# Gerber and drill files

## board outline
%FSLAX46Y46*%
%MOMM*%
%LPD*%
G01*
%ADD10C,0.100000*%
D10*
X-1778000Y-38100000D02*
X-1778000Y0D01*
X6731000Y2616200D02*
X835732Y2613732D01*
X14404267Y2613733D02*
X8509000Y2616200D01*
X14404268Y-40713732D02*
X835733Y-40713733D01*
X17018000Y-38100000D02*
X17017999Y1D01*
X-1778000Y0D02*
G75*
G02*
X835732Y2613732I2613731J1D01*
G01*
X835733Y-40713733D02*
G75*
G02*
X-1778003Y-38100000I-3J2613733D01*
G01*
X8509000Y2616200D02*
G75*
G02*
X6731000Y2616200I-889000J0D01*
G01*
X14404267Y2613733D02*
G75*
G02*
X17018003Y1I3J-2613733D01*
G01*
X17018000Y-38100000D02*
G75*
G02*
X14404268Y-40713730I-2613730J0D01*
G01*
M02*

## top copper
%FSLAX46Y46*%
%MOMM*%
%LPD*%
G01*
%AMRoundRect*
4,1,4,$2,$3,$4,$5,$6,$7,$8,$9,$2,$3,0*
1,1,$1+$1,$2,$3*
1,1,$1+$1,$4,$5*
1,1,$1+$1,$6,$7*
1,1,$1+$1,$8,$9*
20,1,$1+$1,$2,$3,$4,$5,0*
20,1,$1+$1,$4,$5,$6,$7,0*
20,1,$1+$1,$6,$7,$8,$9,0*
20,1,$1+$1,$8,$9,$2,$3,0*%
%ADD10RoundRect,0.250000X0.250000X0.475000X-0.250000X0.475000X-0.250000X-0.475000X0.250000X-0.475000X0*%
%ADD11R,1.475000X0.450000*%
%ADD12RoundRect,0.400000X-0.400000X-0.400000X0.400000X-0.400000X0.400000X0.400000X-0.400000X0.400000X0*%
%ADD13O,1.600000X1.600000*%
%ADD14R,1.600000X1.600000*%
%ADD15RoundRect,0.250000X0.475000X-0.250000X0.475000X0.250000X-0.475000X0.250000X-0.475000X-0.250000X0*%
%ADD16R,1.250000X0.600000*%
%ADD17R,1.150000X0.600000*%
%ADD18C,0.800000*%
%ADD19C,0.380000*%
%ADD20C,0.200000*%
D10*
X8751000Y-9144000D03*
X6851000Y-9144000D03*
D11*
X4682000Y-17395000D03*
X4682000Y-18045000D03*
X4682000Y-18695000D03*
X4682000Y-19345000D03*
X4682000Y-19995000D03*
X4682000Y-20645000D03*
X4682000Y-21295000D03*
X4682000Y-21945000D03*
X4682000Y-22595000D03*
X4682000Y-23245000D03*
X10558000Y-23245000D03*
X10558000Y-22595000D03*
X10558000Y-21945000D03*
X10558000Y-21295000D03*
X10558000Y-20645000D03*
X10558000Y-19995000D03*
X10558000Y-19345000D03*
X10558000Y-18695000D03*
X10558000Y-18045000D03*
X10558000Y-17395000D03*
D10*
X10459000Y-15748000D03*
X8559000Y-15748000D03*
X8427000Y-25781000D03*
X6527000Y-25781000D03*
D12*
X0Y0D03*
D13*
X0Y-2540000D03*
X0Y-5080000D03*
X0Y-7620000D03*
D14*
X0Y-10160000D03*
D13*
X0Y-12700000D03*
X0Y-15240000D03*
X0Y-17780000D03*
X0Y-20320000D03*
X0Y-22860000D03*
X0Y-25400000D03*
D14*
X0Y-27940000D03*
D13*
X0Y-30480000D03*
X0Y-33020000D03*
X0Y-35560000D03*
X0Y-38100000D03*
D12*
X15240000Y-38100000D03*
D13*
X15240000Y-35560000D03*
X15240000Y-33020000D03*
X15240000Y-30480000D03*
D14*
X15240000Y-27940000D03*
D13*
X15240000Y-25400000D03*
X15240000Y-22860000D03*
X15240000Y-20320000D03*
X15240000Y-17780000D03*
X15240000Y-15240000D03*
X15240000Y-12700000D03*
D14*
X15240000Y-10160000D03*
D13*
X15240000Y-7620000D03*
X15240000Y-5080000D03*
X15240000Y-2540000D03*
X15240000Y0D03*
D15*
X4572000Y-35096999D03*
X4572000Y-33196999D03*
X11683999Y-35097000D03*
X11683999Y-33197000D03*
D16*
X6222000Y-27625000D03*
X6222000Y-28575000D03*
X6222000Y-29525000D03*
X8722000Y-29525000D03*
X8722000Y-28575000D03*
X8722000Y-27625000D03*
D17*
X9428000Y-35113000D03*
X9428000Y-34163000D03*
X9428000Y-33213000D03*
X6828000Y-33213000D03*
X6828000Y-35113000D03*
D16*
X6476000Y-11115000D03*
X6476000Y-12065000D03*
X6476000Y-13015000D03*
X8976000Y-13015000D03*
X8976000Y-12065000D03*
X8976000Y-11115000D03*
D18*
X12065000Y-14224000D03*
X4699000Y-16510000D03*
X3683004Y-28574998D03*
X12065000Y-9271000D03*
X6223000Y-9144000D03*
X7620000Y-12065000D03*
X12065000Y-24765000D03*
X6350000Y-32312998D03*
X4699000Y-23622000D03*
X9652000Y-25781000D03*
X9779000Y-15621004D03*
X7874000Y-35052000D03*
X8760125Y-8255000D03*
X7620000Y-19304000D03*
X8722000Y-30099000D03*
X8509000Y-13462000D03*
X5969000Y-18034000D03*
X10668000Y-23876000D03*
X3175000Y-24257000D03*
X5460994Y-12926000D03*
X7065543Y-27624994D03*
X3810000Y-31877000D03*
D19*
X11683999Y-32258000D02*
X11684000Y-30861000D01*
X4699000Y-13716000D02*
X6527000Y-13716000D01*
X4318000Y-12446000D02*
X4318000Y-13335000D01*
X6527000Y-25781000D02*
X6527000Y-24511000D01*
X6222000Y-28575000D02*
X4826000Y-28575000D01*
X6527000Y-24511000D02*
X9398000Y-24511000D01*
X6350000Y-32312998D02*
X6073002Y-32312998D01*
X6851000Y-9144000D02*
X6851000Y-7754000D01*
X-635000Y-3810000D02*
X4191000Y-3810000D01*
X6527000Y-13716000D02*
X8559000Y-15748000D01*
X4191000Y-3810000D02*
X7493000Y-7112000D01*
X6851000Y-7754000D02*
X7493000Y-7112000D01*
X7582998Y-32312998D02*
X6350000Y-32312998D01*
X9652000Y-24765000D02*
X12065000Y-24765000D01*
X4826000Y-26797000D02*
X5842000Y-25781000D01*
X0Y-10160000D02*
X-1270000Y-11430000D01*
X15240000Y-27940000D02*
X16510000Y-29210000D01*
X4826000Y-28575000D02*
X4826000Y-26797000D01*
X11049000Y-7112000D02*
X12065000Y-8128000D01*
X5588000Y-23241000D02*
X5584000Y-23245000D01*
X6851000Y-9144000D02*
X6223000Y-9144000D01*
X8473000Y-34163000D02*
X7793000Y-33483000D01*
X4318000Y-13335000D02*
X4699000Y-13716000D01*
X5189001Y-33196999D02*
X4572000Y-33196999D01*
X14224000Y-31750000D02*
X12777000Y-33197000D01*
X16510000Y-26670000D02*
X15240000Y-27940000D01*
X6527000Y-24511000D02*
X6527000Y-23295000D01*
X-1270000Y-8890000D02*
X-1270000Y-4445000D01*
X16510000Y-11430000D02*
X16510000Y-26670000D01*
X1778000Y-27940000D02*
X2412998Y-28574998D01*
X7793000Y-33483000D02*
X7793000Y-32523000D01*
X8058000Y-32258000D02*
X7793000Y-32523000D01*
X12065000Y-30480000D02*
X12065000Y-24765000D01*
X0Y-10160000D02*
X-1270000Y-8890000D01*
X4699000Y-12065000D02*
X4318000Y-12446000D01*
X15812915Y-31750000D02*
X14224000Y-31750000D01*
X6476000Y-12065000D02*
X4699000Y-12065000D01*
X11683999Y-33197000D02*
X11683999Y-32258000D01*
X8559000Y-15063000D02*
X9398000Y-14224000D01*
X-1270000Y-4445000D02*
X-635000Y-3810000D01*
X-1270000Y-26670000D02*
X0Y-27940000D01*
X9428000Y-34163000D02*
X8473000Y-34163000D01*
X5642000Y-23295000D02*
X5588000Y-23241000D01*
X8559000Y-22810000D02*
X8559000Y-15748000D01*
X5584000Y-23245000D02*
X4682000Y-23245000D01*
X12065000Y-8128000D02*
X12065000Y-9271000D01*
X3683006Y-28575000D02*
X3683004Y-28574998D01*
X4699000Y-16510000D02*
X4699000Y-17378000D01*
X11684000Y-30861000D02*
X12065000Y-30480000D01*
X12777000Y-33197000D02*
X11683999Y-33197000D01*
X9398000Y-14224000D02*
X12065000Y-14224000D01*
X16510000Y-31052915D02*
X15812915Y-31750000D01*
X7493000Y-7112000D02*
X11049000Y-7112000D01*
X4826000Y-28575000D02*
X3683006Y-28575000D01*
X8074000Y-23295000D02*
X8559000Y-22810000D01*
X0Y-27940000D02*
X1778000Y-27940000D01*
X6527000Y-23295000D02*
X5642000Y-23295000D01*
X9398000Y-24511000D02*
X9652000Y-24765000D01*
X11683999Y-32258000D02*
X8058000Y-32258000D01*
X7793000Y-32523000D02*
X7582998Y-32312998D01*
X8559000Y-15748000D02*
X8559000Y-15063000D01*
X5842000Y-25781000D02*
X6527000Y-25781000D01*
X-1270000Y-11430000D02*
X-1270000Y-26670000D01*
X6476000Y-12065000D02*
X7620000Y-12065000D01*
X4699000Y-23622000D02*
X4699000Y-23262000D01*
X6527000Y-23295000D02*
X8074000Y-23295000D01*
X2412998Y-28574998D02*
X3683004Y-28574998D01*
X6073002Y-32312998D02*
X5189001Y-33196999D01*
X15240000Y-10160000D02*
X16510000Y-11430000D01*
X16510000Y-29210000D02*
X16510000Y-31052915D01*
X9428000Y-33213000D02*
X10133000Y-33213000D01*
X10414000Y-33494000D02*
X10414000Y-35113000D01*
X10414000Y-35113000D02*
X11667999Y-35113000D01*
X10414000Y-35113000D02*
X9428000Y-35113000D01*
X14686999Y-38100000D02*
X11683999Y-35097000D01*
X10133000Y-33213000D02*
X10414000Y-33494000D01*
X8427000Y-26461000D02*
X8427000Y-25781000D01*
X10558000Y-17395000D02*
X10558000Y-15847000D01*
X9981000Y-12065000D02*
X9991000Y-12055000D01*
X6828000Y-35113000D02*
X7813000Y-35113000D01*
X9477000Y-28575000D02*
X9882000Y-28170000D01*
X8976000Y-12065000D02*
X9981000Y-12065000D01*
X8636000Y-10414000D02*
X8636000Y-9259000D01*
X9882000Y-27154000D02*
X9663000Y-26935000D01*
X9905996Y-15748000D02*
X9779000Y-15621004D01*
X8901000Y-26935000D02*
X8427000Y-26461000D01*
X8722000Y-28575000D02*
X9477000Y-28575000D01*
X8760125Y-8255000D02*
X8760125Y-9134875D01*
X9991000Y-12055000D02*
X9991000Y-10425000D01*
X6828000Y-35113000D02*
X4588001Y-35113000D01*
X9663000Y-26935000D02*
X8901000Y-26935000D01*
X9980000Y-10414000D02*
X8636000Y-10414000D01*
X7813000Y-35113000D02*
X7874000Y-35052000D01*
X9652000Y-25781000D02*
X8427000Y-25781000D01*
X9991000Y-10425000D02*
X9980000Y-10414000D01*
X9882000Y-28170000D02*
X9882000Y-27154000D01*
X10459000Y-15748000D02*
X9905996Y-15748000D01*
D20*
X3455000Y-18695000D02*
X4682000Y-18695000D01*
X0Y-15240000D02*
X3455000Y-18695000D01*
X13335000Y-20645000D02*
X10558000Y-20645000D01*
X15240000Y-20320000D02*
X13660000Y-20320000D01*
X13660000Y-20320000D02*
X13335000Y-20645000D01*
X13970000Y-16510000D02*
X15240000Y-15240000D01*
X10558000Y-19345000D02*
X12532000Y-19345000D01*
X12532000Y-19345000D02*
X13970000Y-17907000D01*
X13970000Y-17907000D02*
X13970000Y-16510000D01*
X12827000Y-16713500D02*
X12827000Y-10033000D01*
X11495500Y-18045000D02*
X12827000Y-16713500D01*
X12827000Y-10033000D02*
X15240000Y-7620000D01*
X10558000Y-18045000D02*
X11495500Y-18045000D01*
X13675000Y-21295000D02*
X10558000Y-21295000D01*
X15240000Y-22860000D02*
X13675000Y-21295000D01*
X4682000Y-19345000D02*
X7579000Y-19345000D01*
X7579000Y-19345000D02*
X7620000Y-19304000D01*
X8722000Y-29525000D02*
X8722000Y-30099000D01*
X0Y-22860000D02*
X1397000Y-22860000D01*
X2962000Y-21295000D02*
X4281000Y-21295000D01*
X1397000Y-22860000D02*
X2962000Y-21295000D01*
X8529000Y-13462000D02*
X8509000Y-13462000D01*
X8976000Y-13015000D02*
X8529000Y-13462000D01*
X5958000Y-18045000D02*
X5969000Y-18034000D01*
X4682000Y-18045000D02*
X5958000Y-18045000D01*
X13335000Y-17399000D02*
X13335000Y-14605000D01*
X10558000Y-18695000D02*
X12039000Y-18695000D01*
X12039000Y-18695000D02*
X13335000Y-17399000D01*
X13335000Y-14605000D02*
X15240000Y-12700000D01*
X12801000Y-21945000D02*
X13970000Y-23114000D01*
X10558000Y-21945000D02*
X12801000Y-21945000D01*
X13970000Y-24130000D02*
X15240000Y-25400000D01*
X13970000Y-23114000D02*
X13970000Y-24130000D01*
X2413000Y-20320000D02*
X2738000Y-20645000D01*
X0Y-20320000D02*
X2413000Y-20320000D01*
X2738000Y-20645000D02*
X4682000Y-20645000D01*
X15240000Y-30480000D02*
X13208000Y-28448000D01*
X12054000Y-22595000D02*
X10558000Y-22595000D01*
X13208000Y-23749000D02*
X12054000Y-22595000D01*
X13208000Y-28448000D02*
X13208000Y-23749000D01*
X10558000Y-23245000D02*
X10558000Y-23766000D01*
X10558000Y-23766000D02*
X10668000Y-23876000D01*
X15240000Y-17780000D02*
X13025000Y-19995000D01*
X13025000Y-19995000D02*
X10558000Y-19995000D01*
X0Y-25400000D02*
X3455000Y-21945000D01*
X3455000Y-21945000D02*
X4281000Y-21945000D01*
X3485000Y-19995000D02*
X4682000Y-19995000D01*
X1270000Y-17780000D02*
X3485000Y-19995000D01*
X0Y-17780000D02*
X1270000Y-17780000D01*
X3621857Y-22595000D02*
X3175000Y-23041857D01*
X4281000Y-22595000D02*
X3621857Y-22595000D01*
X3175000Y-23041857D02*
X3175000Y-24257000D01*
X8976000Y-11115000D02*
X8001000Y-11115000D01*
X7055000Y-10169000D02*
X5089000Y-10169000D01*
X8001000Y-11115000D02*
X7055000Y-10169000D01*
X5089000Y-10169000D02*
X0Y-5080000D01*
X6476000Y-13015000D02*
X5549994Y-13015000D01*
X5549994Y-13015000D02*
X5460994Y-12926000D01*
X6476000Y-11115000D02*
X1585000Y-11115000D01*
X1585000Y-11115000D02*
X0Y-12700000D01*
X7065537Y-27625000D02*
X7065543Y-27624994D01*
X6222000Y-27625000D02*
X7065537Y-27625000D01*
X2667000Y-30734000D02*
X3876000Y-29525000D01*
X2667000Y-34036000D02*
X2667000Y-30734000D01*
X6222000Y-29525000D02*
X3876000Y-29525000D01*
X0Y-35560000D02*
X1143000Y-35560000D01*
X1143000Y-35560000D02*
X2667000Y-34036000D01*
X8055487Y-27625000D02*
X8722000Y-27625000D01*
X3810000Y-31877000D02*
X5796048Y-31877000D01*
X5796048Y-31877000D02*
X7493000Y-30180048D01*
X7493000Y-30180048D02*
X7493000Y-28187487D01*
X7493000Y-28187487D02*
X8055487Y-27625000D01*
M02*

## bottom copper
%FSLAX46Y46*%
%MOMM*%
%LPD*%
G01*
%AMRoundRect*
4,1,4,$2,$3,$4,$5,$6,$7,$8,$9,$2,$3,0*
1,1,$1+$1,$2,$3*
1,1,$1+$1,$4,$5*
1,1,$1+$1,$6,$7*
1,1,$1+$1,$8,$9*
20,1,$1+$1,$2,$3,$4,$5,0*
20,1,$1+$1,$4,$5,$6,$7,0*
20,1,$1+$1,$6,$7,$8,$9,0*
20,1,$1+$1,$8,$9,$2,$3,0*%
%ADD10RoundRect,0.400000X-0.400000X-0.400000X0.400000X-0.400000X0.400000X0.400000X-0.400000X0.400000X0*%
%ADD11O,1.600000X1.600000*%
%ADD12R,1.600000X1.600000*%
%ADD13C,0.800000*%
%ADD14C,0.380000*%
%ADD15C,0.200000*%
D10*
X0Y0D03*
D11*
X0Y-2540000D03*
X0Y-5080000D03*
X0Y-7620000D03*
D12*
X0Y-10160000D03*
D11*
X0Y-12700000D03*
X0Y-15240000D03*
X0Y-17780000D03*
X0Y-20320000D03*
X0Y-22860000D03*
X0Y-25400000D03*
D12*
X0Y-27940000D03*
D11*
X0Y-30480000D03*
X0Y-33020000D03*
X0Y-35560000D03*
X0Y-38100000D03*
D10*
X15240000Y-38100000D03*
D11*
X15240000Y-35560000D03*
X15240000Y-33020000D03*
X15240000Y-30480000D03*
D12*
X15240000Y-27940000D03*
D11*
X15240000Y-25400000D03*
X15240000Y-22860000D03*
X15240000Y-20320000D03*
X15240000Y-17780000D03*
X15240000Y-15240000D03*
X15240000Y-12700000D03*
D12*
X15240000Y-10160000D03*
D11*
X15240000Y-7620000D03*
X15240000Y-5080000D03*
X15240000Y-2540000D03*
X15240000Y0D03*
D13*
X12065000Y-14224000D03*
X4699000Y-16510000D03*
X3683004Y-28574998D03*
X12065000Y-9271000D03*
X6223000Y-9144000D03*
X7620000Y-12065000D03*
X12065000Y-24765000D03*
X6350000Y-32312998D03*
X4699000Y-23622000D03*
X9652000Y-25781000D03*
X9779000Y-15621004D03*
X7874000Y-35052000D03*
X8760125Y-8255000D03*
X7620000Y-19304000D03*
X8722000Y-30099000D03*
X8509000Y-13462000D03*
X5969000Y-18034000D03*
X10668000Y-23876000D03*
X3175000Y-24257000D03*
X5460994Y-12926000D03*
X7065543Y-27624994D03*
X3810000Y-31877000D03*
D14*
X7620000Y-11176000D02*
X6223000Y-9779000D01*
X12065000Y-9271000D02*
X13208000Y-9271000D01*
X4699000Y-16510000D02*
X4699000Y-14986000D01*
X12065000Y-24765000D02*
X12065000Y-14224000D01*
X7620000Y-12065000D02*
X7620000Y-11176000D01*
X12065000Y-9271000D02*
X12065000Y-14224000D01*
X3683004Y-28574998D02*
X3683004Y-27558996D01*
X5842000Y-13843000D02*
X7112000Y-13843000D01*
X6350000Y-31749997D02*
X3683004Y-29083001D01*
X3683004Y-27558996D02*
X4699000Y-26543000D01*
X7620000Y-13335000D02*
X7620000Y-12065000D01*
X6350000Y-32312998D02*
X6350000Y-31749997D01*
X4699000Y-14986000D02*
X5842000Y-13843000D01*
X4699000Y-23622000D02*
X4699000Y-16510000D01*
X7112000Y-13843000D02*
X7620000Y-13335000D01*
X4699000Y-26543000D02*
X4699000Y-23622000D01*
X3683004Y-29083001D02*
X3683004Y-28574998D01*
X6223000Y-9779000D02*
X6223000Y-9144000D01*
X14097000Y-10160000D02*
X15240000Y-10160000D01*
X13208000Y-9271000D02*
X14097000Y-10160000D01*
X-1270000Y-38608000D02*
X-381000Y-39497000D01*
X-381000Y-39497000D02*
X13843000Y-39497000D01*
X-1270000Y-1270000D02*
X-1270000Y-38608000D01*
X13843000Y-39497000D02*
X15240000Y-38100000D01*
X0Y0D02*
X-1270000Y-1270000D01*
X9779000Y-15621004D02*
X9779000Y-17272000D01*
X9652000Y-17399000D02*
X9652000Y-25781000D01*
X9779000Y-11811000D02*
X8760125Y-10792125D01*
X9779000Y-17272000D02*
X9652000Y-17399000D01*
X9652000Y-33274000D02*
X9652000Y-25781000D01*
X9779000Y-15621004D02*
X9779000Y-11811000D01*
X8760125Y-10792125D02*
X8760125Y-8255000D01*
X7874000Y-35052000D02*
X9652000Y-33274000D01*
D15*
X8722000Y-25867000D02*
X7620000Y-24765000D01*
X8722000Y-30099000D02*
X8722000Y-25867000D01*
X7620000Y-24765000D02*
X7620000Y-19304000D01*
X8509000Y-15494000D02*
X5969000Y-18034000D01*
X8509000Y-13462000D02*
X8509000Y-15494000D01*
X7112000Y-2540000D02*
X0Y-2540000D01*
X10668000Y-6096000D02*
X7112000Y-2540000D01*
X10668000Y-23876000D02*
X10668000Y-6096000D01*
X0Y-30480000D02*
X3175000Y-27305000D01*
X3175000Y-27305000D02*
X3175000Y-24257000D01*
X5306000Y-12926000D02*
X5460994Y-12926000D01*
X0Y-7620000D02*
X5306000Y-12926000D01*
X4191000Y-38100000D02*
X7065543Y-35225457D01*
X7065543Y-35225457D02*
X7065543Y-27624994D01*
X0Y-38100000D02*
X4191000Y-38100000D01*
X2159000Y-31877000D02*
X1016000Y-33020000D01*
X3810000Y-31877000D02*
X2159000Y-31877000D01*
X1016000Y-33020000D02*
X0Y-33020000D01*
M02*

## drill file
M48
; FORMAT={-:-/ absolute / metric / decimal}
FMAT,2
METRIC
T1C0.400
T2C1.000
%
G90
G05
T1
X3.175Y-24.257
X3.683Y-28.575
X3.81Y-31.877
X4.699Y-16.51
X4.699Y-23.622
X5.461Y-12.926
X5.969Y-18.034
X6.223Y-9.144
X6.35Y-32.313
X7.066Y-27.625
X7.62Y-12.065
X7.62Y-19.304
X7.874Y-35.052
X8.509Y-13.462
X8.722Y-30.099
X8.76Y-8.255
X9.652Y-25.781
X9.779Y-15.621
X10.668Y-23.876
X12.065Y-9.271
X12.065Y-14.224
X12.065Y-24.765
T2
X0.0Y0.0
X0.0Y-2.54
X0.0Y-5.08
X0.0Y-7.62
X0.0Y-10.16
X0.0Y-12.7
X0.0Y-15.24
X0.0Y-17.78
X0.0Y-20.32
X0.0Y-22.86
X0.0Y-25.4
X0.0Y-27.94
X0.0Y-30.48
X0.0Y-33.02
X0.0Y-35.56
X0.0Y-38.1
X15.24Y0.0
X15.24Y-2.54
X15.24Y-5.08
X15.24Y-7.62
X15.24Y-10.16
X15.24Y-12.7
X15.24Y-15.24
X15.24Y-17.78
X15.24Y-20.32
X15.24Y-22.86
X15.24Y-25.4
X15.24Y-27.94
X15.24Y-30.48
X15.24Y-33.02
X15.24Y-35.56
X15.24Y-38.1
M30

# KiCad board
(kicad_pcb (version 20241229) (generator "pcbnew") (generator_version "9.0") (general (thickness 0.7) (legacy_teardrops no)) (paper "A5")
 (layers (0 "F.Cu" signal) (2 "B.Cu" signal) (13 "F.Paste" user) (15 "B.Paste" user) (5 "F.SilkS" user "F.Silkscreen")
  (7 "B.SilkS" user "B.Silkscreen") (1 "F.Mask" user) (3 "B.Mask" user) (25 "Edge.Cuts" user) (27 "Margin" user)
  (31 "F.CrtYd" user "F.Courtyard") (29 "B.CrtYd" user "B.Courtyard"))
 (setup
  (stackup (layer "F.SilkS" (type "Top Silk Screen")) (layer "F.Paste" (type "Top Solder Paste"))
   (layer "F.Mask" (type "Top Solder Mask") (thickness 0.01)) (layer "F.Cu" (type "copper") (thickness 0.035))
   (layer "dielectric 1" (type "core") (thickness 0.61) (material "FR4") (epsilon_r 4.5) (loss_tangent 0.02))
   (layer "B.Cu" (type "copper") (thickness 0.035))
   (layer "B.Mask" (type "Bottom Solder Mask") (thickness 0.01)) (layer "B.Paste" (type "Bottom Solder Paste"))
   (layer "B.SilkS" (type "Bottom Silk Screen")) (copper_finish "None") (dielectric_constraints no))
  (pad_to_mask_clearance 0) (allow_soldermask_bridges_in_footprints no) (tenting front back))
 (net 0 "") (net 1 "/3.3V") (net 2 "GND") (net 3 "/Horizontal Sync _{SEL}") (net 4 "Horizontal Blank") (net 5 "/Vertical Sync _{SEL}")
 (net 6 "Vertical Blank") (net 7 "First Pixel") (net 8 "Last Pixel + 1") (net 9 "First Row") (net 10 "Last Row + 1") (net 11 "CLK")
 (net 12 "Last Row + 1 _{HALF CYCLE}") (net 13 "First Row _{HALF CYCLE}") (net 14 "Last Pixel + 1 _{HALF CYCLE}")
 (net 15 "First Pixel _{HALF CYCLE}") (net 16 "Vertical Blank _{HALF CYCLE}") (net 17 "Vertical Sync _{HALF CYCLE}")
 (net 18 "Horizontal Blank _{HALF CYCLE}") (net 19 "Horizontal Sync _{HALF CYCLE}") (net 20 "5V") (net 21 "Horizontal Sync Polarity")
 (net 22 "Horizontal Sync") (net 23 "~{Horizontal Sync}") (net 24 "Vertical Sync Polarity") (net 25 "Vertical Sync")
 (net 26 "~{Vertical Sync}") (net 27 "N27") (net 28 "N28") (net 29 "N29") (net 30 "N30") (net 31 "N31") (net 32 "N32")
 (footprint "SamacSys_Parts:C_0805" (layer "F.Cu") (at 7.817 9.144 90)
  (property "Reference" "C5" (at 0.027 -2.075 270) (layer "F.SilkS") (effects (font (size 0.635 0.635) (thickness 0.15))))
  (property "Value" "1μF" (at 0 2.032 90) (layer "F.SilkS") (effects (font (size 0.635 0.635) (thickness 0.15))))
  (pad "1" smd roundrect (at 0 0.934 180) (size 1 1.45) (layers "F.Cu" "F.Mask" "F.Paste") (roundrect_rratio 0.25) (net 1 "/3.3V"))
  (pad "2" smd roundrect (at 0 -0.966 180) (size 1 1.45) (layers "F.Cu" "F.Mask" "F.Paste") (roundrect_rratio 0.25) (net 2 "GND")))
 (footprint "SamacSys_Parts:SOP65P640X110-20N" (layer "F.Cu") (at 7.62 20.32)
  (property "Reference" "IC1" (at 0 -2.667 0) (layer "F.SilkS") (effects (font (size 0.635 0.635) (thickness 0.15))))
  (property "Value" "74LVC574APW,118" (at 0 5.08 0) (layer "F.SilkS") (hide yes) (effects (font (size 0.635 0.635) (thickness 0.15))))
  (pad "1" smd rect (at -2.938 -2.925 90) (size 0.45 1.475) (layers "F.Cu" "F.Mask" "F.Paste") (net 2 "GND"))
  (pad "2" smd rect (at -2.938 -2.275 90) (size 0.45 1.475) (layers "F.Cu" "F.Mask" "F.Paste") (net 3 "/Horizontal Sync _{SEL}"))
  (pad "3" smd rect (at -2.938 -1.625 90) (size 0.45 1.475) (layers "F.Cu" "F.Mask" "F.Paste") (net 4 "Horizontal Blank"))
  (pad "4" smd rect (at -2.938 -0.975 90) (size 0.45 1.475) (layers "F.Cu" "F.Mask" "F.Paste") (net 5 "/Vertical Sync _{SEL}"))
  (pad "5" smd rect (at -2.938 -0.325 90) (size 0.45 1.475) (layers "F.Cu" "F.Mask" "F.Paste") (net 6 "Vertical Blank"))
  (pad "6" smd rect (at -2.938 0.325 90) (size 0.45 1.475) (layers "F.Cu" "F.Mask" "F.Paste") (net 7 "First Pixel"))
  (pad "7" smd rect (at -2.938 0.975 90) (size 0.45 1.475) (layers "F.Cu" "F.Mask" "F.Paste") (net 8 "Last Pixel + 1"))
  (pad "8" smd rect (at -2.938 1.625 90) (size 0.45 1.475) (layers "F.Cu" "F.Mask" "F.Paste") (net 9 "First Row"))
  (pad "9" smd rect (at -2.938 2.275 90) (size 0.45 1.475) (layers "F.Cu" "F.Mask" "F.Paste") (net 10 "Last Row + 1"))
  (pad "10" smd rect (at -2.938 2.925 90) (size 0.45 1.475) (layers "F.Cu" "F.Mask" "F.Paste") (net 2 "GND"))
  (pad "11" smd rect (at 2.938 2.925 90) (size 0.45 1.475) (layers "F.Cu" "F.Mask" "F.Paste") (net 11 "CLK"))
  (pad "12" smd rect (at 2.938 2.275 90) (size 0.45 1.475) (layers "F.Cu" "F.Mask" "F.Paste") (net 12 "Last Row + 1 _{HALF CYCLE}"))
  (pad "13" smd rect (at 2.938 1.625 90) (size 0.45 1.475) (layers "F.Cu" "F.Mask" "F.Paste") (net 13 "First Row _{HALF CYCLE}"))
  (pad "14" smd rect (at 2.938 0.975 90) (size 0.45 1.475) (layers "F.Cu" "F.Mask" "F.Paste") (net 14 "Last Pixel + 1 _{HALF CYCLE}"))
  (pad "15" smd rect (at 2.938 0.325 90) (size 0.45 1.475) (layers "F.Cu" "F.Mask" "F.Paste") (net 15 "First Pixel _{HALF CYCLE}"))
  (pad "16" smd rect (at 2.938 -0.325 90) (size 0.45 1.475) (layers "F.Cu" "F.Mask" "F.Paste") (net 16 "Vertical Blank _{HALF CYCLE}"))
  (pad "17" smd rect (at 2.938 -0.975 90) (size 0.45 1.475) (layers "F.Cu" "F.Mask" "F.Paste") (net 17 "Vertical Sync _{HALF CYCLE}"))
  (pad "18" smd rect (at 2.938 -1.625 90) (size 0.45 1.475) (layers "F.Cu" "F.Mask" "F.Paste") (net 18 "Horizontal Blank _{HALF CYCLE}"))
  (pad "19" smd rect (at 2.938 -2.275 90) (size 0.45 1.475) (layers "F.Cu" "F.Mask" "F.Paste") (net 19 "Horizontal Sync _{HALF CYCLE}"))
  (pad "20" smd rect (at 2.938 -2.925 90) (size 0.45 1.475) (layers "F.Cu" "F.Mask" "F.Paste") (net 1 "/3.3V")))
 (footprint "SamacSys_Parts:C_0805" (layer "F.Cu") (at 9.525 15.748 90)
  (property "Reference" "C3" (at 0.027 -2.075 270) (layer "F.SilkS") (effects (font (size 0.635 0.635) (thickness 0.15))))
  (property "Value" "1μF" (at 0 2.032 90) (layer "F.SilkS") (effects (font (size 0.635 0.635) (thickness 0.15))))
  (pad "1" smd roundrect (at 0 0.934 180) (size 1 1.45) (layers "F.Cu" "F.Mask" "F.Paste") (roundrect_rratio 0.25) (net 1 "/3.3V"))
  (pad "2" smd roundrect (at 0 -0.966 180) (size 1 1.45) (layers "F.Cu" "F.Mask" "F.Paste") (roundrect_rratio 0.25) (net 2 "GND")))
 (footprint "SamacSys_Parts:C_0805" (layer "F.Cu") (at 7.493 25.781 90)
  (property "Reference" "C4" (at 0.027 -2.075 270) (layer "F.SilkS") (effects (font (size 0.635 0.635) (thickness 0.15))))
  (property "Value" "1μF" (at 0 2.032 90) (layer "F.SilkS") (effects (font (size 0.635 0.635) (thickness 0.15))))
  (pad "1" smd roundrect (at 0 0.934 180) (size 1 1.45) (layers "F.Cu" "F.Mask" "F.Paste") (roundrect_rratio 0.25) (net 1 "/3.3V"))
  (pad "2" smd roundrect (at 0 -0.966 180) (size 1 1.45) (layers "F.Cu" "F.Mask" "F.Paste") (roundrect_rratio 0.25) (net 2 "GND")))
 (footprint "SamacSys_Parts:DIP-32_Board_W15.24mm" (layer "F.Cu") (at 0 0)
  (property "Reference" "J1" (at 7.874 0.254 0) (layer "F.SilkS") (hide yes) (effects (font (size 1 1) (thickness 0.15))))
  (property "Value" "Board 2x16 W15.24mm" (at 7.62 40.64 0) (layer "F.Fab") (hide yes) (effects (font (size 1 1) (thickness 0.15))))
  (fp_line (start -1.778 38.1) (end -1.778 0) (stroke (width 0.1) (type solid)) (layer "Edge.Cuts"))
  (fp_line (start 6.731 -2.6162) (end 0.835732 -2.613732) (stroke (width 0.1) (type solid)) (layer "Edge.Cuts"))
  (fp_line (start 14.404267 -2.613733) (end 8.509 -2.6162) (stroke (width 0.1) (type solid)) (layer "Edge.Cuts"))
  (fp_line (start 14.404268 40.713732) (end 0.835733 40.713733) (stroke (width 0.1) (type solid)) (layer "Edge.Cuts"))
  (fp_line (start 17.018 38.1) (end 17.017999 -0.000001) (stroke (width 0.1) (type solid)) (layer "Edge.Cuts"))
  (fp_arc (start -1.778 0) (mid -1.012456 -1.848188) (end 0.835732 -2.613732) (stroke (width 0.1) (type solid)) (layer "Edge.Cuts"))
  (fp_arc (start 0.835733 40.713733) (mid -1.012456 39.948189) (end -1.778 38.1) (stroke (width 0.1) (type solid)) (layer "Edge.Cuts"))
  (fp_arc (start 8.509 -2.6162) (mid 7.62 -1.7272) (end 6.731 -2.6162) (stroke (width 0.1) (type default)) (layer "Edge.Cuts"))
  (fp_arc (start 14.404267 -2.613733) (mid 16.252455 -1.848189) (end 17.017999 -0.000001) (stroke (width 0.1) (type solid))
   (layer "Edge.Cuts"))
  (fp_arc (start 17.018 38.1) (mid 16.252455 39.948187) (end 14.404268 40.713732) (stroke (width 0.1) (type solid)) (layer "Edge.Cuts"))
  (pad "1" thru_hole roundrect (at 0 0) (size 1.6 1.6) (drill 1) (layers "*.Cu" "*.Mask") (remove_unused_layers no) (roundrect_rratio 0.25)
   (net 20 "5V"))
  (pad "2" thru_hole oval (at 0 2.54) (size 1.6 1.6) (drill 1) (layers "*.Cu" "*.Mask") (remove_unused_layers no) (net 11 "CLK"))
  (pad "3" thru_hole oval (at 0 5.08) (size 1.6 1.6) (drill 1) (layers "*.Cu" "*.Mask") (remove_unused_layers no)
   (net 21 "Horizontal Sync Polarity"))
  (pad "4" thru_hole oval (at 0 7.62) (size 1.6 1.6) (drill 1) (layers "*.Cu" "*.Mask") (remove_unused_layers no) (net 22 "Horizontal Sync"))
  (pad "5" thru_hole rect (at 0 10.16) (size 1.6 1.6) (drill 1) (layers "*.Cu" "*.Mask") (remove_unused_layers no) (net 2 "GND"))
  (pad "6" thru_hole oval (at 0 12.7) (size 1.6 1.6) (drill 1) (layers "*.Cu" "*.Mask") (remove_unused_layers no)
   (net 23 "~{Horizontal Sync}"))
  (pad "7" thru_hole oval (at 0 15.24) (size 1.6 1.6) (drill 1) (layers "*.Cu" "*.Mask") (remove_unused_layers no)
   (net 4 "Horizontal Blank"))
  (pad "8" thru_hole oval (at 0 17.78) (size 1.6 1.6) (drill 1) (layers "*.Cu" "*.Mask") (remove_unused_layers no) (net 6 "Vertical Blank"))
  (pad "9" thru_hole oval (at 0 20.32) (size 1.6 1.6) (drill 1) (layers "*.Cu" "*.Mask") (remove_unused_layers no) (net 7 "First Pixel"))
  (pad "10" thru_hole oval (at 0 22.86) (size 1.6 1.6) (drill 1) (layers "*.Cu" "*.Mask") (remove_unused_layers no) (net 8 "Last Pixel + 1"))
  (pad "11" thru_hole oval (at 0 25.4) (size 1.6 1.6) (drill 1) (layers "*.Cu" "*.Mask") (remove_unused_layers no) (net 9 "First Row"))
  (pad "12" thru_hole rect (at 0 27.94) (size 1.6 1.6) (drill 1) (layers "*.Cu" "*.Mask") (remove_unused_layers no) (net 2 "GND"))
  (pad "13" thru_hole oval (at 0 30.48) (size 1.6 1.6) (drill 1) (layers "*.Cu" "*.Mask") (remove_unused_layers no) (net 10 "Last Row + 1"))
  (pad "14" thru_hole oval (at 0 33.02) (size 1.6 1.6) (drill 1) (layers "*.Cu" "*.Mask") (remove_unused_layers no)
   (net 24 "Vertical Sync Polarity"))
  (pad "15" thru_hole oval (at 0 35.56) (size 1.6 1.6) (drill 1) (layers "*.Cu" "*.Mask") (remove_unused_layers no) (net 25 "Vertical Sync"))
  (pad "16" thru_hole oval (at 0 38.1) (size 1.6 1.6) (drill 1) (layers "*.Cu" "*.Mask") (remove_unused_layers no)
   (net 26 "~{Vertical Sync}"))
  (pad "17" thru_hole roundrect (at 15.24 38.1) (size 1.6 1.6) (drill 1) (layers "*.Cu" "*.Mask") (remove_unused_layers no)
   (roundrect_rratio 0.25) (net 20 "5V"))
  (pad "18" thru_hole oval (at 15.24 35.56 180) (size 1.6 1.6) (drill 1) (layers "*.Cu" "*.Mask") (remove_unused_layers no) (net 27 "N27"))
  (pad "19" thru_hole oval (at 15.24 33.02 180) (size 1.6 1.6) (drill 1) (layers "*.Cu" "*.Mask") (remove_unused_layers no) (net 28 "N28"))
  (pad "20" thru_hole oval (at 15.24 30.48 180) (size 1.6 1.6) (drill 1) (layers "*.Cu" "*.Mask") (remove_unused_layers no)
   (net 12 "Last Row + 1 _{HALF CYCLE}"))
  (pad "21" thru_hole rect (at 15.24 27.94) (size 1.6 1.6) (drill 1) (layers "*.Cu" "*.Mask") (remove_unused_layers no) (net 2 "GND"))
  (pad "22" thru_hole oval (at 15.24 25.4) (size 1.6 1.6) (drill 1) (layers "*.Cu" "*.Mask") (remove_unused_layers no)
   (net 13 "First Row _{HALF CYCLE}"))
  (pad "23" thru_hole oval (at 15.24 22.86) (size 1.6 1.6) (drill 1) (layers "*.Cu" "*.Mask") (remove_unused_layers no)
   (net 14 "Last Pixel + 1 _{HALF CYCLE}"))
  (pad "24" thru_hole oval (at 15.24 20.32) (size 1.6 1.6) (drill 1) (layers "*.Cu" "*.Mask") (remove_unused_layers no)
   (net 15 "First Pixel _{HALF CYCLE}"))
  (pad "25" thru_hole oval (at 15.24 17.78) (size 1.6 1.6) (drill 1) (layers "*.Cu" "*.Mask") (remove_unused_layers no)
   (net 16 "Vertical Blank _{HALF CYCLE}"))
  (pad "26" thru_hole oval (at 15.24 15.24) (size 1.6 1.6) (drill 1) (layers "*.Cu" "*.Mask") (remove_unused_layers no)
   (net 17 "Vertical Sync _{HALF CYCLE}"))
  (pad "27" thru_hole oval (at 15.24 12.7) (size 1.6 1.6) (drill 1) (layers "*.Cu" "*.Mask") (remove_unused_layers no)
   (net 18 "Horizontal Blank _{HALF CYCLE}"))
  (pad "28" thru_hole rect (at 15.24 10.16) (size 1.6 1.6) (drill 1) (layers "*.Cu" "*.Mask") (remove_unused_layers no) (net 2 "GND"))
  (pad "29" thru_hole oval (at 15.24 7.62) (size 1.6 1.6) (drill 1) (layers "*.Cu" "*.Mask") (remove_unused_layers no)
   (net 19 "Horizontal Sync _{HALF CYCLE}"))
  (pad "30" thru_hole oval (at 15.24 5.08) (size 1.6 1.6) (drill 1) (layers "*.Cu" "*.Mask") (remove_unused_layers no) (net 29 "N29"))
  (pad "31" thru_hole oval (at 15.24 2.54) (size 1.6 1.6) (drill 1) (layers "*.Cu" "*.Mask") (remove_unused_layers no) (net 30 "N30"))
  (pad "32" thru_hole oval (at 15.24 0) (size 1.6 1.6) (drill 1) (layers "*.Cu" "*.Mask") (remove_unused_layers no) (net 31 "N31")))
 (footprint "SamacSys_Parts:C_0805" (layer "F.Cu") (at 4.572 34.162999)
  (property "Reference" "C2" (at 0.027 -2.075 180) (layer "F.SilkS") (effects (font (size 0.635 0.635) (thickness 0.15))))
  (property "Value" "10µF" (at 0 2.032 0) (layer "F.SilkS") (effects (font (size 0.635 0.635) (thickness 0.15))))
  (pad "1" smd roundrect (at 0 0.934 90) (size 1 1.45) (layers "F.Cu" "F.Mask" "F.Paste") (roundrect_rratio 0.25) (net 1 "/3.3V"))
  (pad "2" smd roundrect (at 0 -0.966 90) (size 1 1.45) (layers "F.Cu" "F.Mask" "F.Paste") (roundrect_rratio 0.25) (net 2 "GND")))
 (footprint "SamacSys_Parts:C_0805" (layer "F.Cu") (at 11.683999 34.163)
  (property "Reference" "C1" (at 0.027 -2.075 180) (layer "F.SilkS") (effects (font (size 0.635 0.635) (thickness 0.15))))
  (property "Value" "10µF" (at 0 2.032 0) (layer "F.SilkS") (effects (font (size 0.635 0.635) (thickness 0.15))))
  (pad "1" smd roundrect (at 0 0.934 90) (size 1 1.45) (layers "F.Cu" "F.Mask" "F.Paste") (roundrect_rratio 0.25) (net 20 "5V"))
  (pad "2" smd roundrect (at 0 -0.966 90) (size 1 1.45) (layers "F.Cu" "F.Mask" "F.Paste") (roundrect_rratio 0.25) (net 2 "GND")))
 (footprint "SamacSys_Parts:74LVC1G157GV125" (layer "F.Cu") (at 7.493 28.575)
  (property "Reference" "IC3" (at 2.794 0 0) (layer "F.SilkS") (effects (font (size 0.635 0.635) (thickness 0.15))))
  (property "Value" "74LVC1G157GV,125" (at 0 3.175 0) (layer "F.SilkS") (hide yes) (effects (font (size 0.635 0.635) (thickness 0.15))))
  (pad "1" smd rect (at -1.271 -0.95 90) (size 0.6 1.25) (layers "F.Cu" "F.Mask" "F.Paste") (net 26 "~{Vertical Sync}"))
  (pad "2" smd rect (at -1.271 0 90) (size 0.6 1.25) (layers "F.Cu" "F.Mask" "F.Paste") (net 2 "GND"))
  (pad "3" smd rect (at -1.271 0.95 90) (size 0.6 1.25) (layers "F.Cu" "F.Mask" "F.Paste") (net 25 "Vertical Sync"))
  (pad "4" smd rect (at 1.229 0.95 90) (size 0.6 1.25) (layers "F.Cu" "F.Mask" "F.Paste") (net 5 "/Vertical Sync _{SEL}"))
  (pad "5" smd rect (at 1.229 0 90) (size 0.6 1.25) (layers "F.Cu" "F.Mask" "F.Paste") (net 1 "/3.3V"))
  (pad "6" smd rect (at 1.229 -0.95 90) (size 0.6 1.25) (layers "F.Cu" "F.Mask" "F.Paste") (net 24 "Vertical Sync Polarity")))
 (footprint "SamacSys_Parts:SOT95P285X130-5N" (layer "F.Cu") (at 8.128 34.163 180)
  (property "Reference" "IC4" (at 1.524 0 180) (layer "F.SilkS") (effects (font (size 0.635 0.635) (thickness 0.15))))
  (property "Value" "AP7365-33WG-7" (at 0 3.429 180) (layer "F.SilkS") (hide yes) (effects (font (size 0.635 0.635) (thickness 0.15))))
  (pad "1" smd rect (at -1.3 -0.95 270) (size 0.6 1.15) (layers "F.Cu" "F.Mask" "F.Paste") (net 20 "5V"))
  (pad "2" smd rect (at -1.3 0 270) (size 0.6 1.15) (layers "F.Cu" "F.Mask" "F.Paste") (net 2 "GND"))
  (pad "3" smd rect (at -1.3 0.95 270) (size 0.6 1.15) (layers "F.Cu" "F.Mask" "F.Paste") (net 20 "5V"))
  (pad "4" smd rect (at 1.3 0.95 270) (size 0.6 1.15) (layers "F.Cu" "F.Mask" "F.Paste") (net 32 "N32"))
  (pad "5" smd rect (at 1.3 -0.95 270) (size 0.6 1.15) (layers "F.Cu" "F.Mask" "F.Paste") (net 1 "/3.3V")))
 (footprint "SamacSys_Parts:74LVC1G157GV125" (layer "F.Cu") (at 7.747 12.065)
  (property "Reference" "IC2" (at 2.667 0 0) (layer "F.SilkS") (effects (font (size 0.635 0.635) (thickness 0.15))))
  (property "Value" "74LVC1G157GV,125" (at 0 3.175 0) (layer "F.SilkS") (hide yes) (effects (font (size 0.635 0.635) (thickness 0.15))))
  (pad "1" smd rect (at -1.271 -0.95 90) (size 0.6 1.25) (layers "F.Cu" "F.Mask" "F.Paste") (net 23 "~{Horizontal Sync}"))
  (pad "2" smd rect (at -1.271 0 90) (size 0.6 1.25) (layers "F.Cu" "F.Mask" "F.Paste") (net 2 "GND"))
  (pad "3" smd rect (at -1.271 0.95 90) (size 0.6 1.25) (layers "F.Cu" "F.Mask" "F.Paste") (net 22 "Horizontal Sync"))
  (pad "4" smd rect (at 1.229 0.95 90) (size 0.6 1.25) (layers "F.Cu" "F.Mask" "F.Paste") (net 3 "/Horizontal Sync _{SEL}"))
  (pad "5" smd rect (at 1.229 0 90) (size 0.6 1.25) (layers "F.Cu" "F.Mask" "F.Paste") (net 1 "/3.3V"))
  (pad "6" smd rect (at 1.229 -0.95 90) (size 0.6 1.25) (layers "F.Cu" "F.Mask" "F.Paste") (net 21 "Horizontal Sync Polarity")))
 (segment (start 11.683999 32.258) (end 11.684 30.861) (width 0.38) (layer "F.Cu") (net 2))
 (segment (start 4.699 13.716) (end 6.527 13.716) (width 0.38) (layer "F.Cu") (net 2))
 (segment (start 4.318 12.446) (end 4.318 13.335) (width 0.38) (layer "F.Cu") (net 2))
 (segment (start 6.527 25.781) (end 6.527 24.511) (width 0.38) (layer "F.Cu") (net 2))
 (segment (start 6.222 28.575) (end 4.826 28.575) (width 0.38) (layer "F.Cu") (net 2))
 (segment (start 6.527 24.511) (end 9.398 24.511) (width 0.38) (layer "F.Cu") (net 2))
 (segment (start 6.35 32.312998) (end 6.073002 32.312998) (width 0.38) (layer "F.Cu") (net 2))
 (segment (start 6.851 9.144) (end 6.851 7.754) (width 0.38) (layer "F.Cu") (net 2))
 (segment (start -0.635 3.81) (end 4.191 3.81) (width 0.38) (layer "F.Cu") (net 2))
 (segment (start 6.527 13.716) (end 8.559 15.748) (width 0.38) (layer "F.Cu") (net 2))
 (segment (start 4.191 3.81) (end 7.493 7.112) (width 0.38) (layer "F.Cu") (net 2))
 (segment (start 6.851 7.754) (end 7.493 7.112) (width 0.38) (layer "F.Cu") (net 2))
 (segment (start 7.582998 32.312998) (end 6.35 32.312998) (width 0.38) (layer "F.Cu") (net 2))
 (segment (start 9.652 24.765) (end 12.065 24.765) (width 0.38) (layer "F.Cu") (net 2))
 (segment (start 4.826 26.797) (end 5.842 25.781) (width 0.38) (layer "F.Cu") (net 2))
 (segment (start 0 10.16) (end -1.27 11.43) (width 0.38) (layer "F.Cu") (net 2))
 (segment (start 15.24 27.94) (end 16.51 29.21) (width 0.38) (layer "F.Cu") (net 2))
 (segment (start 4.826 28.575) (end 4.826 26.797) (width 0.38) (layer "F.Cu") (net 2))
 (segment (start 11.049 7.112) (end 12.065 8.128) (width 0.38) (layer "F.Cu") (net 2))
 (segment (start 5.588 23.241) (end 5.584 23.245) (width 0.38) (layer "F.Cu") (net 2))
 (segment (start 6.851 9.144) (end 6.223 9.144) (width 0.38) (layer "F.Cu") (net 2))
 (segment (start 8.473 34.163) (end 7.793 33.483) (width 0.38) (layer "F.Cu") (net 2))
 (segment (start 4.318 13.335) (end 4.699 13.716) (width 0.38) (layer "F.Cu") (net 2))
 (segment (start 5.189001 33.196999) (end 4.572 33.196999) (width 0.38) (layer "F.Cu") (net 2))
 (segment (start 14.224 31.75) (end 12.777 33.197) (width 0.38) (layer "F.Cu") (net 2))
 (segment (start 16.51 26.67) (end 15.24 27.94) (width 0.38) (layer "F.Cu") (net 2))
 (segment (start 6.527 24.511) (end 6.527 23.295) (width 0.38) (layer "F.Cu") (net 2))
 (segment (start -1.27 8.89) (end -1.27 4.445) (width 0.38) (layer "F.Cu") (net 2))
 (segment (start 16.51 11.43) (end 16.51 26.67) (width 0.38) (layer "F.Cu") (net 2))
 (segment (start 1.778 27.94) (end 2.412998 28.574998) (width 0.38) (layer "F.Cu") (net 2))
 (segment (start 7.793 33.483) (end 7.793 32.523) (width 0.38) (layer "F.Cu") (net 2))
 (segment (start 8.058 32.258) (end 7.793 32.523) (width 0.38) (layer "F.Cu") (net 2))
 (segment (start 12.065 30.48) (end 12.065 24.765) (width 0.38) (layer "F.Cu") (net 2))
 (segment (start 0 10.16) (end -1.27 8.89) (width 0.38) (layer "F.Cu") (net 2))
 (segment (start 4.699 12.065) (end 4.318 12.446) (width 0.38) (layer "F.Cu") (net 2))
 (segment (start 15.812915 31.75) (end 14.224 31.75) (width 0.38) (layer "F.Cu") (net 2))
 (segment (start 6.476 12.065) (end 4.699 12.065) (width 0.38) (layer "F.Cu") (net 2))
 (segment (start 11.683999 33.197) (end 11.683999 32.258) (width 0.38) (layer "F.Cu") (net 2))
 (segment (start 8.559 15.063) (end 9.398 14.224) (width 0.38) (layer "F.Cu") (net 2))
 (segment (start -1.27 4.445) (end -0.635 3.81) (width 0.38) (layer "F.Cu") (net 2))
 (segment (start -1.27 26.67) (end 0 27.94) (width 0.38) (layer "F.Cu") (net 2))
 (segment (start 9.428 34.163) (end 8.473 34.163) (width 0.38) (layer "F.Cu") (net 2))
 (segment (start 5.642 23.295) (end 5.588 23.241) (width 0.38) (layer "F.Cu") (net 2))
 (segment (start 8.559 22.81) (end 8.559 15.748) (width 0.38) (layer "F.Cu") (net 2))
 (segment (start 5.584 23.245) (end 4.682 23.245) (width 0.38) (layer "F.Cu") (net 2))
 (segment (start 12.065 8.128) (end 12.065 9.271) (width 0.38) (layer "F.Cu") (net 2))
 (segment (start 3.683006 28.575) (end 3.683004 28.574998) (width 0.38) (layer "F.Cu") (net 2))
 (segment (start 4.699 16.51) (end 4.699 17.378) (width 0.38) (layer "F.Cu") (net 2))
 (segment (start 11.684 30.861) (end 12.065 30.48) (width 0.38) (layer "F.Cu") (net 2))
 (segment (start 12.777 33.197) (end 11.683999 33.197) (width 0.38) (layer "F.Cu") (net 2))
 (segment (start 9.398 14.224) (end 12.065 14.224) (width 0.38) (layer "F.Cu") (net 2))
 (segment (start 16.51 31.052915) (end 15.812915 31.75) (width 0.38) (layer "F.Cu") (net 2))
 (segment (start 7.493 7.112) (end 11.049 7.112) (width 0.38) (layer "F.Cu") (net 2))
 (segment (start 4.826 28.575) (end 3.683006 28.575) (width 0.38) (layer "F.Cu") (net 2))
 (segment (start 8.074 23.295) (end 8.559 22.81) (width 0.38) (layer "F.Cu") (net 2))
 (segment (start 0 27.94) (end 1.778 27.94) (width 0.38) (layer "F.Cu") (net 2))
 (segment (start 6.527 23.295) (end 5.642 23.295) (width 0.38) (layer "F.Cu") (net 2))
 (segment (start 9.398 24.511) (end 9.652 24.765) (width 0.38) (layer "F.Cu") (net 2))
 (segment (start 11.683999 32.258) (end 8.058 32.258) (width 0.38) (layer "F.Cu") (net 2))
 (segment (start 7.793 32.523) (end 7.582998 32.312998) (width 0.38) (layer "F.Cu") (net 2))
 (segment (start 8.559 15.748) (end 8.559 15.063) (width 0.38) (layer "F.Cu") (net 2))
 (segment (start 5.842 25.781) (end 6.527 25.781) (width 0.38) (layer "F.Cu") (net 2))
 (segment (start -1.27 11.43) (end -1.27 26.67) (width 0.38) (layer "F.Cu") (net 2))
 (segment (start 6.476 12.065) (end 7.62 12.065) (width 0.38) (layer "F.Cu") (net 2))
 (segment (start 4.699 23.622) (end 4.699 23.262) (width 0.38) (layer "F.Cu") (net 2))
 (segment (start 6.527 23.295) (end 8.074 23.295) (width 0.38) (layer "F.Cu") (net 2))
 (segment (start 2.412998 28.574998) (end 3.683004 28.574998) (width 0.38) (layer "F.Cu") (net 2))
 (segment (start 6.073002 32.312998) (end 5.189001 33.196999) (width 0.38) (layer "F.Cu") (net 2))
 (segment (start 15.24 10.16) (end 16.51 11.43) (width 0.38) (layer "F.Cu") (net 2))
 (segment (start 16.51 29.21) (end 16.51 31.052915) (width 0.38) (layer "F.Cu") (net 2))
 (via (at 12.065 14.224) (size 0.8) (drill 0.4) (layers "F.Cu" "B.Cu") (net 2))
 (via (at 4.699 16.51) (size 0.8) (drill 0.4) (layers "F.Cu" "B.Cu") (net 2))
 (via (at 3.683004 28.574998) (size 0.8) (drill 0.4) (layers "F.Cu" "B.Cu") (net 2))
 (via (at 12.065 9.271) (size 0.8) (drill 0.4) (layers "F.Cu" "B.Cu") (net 2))
 (via (at 6.223 9.144) (size 0.8) (drill 0.4) (layers "F.Cu" "B.Cu") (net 2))
 (via (at 7.62 12.065) (size 0.8) (drill 0.4) (layers "F.Cu" "B.Cu") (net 2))
 (via (at 12.065 24.765) (size 0.8) (drill 0.4) (layers "F.Cu" "B.Cu") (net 2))
 (via (at 6.35 32.312998) (size 0.8) (drill 0.4) (layers "F.Cu" "B.Cu") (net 2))
 (via (at 4.699 23.622) (size 0.8) (drill 0.4) (layers "F.Cu" "B.Cu") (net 2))
 (segment (start 7.62 11.176) (end 6.223 9.779) (width 0.38) (layer "B.Cu") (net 2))
 (segment (start 12.065 9.271) (end 13.208 9.271) (width 0.38) (layer "B.Cu") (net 2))
 (segment (start 4.699 16.51) (end 4.699 14.986) (width 0.38) (layer "B.Cu") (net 2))
 (segment (start 12.065 24.765) (end 12.065 14.224) (width 0.38) (layer "B.Cu") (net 2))
 (segment (start 7.62 12.065) (end 7.62 11.176) (width 0.38) (layer "B.Cu") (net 2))
 (segment (start 12.065 9.271) (end 12.065 14.224) (width 0.38) (layer "B.Cu") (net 2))
 (segment (start 3.683004 28.574998) (end 3.683004 27.558996) (width 0.38) (layer "B.Cu") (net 2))
 (segment (start 5.842 13.843) (end 7.112 13.843) (width 0.38) (layer "B.Cu") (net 2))
 (segment (start 6.35 31.749997) (end 3.683004 29.083001) (width 0.38) (layer "B.Cu") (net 2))
 (segment (start 3.683004 27.558996) (end 4.699 26.543) (width 0.38) (layer "B.Cu") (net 2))
 (segment (start 7.62 13.335) (end 7.62 12.065) (width 0.38) (layer "B.Cu") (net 2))
 (segment (start 6.35 32.312998) (end 6.35 31.749997) (width 0.38) (layer "B.Cu") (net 2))
 (segment (start 4.699 14.986) (end 5.842 13.843) (width 0.38) (layer "B.Cu") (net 2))
 (segment (start 4.699 23.622) (end 4.699 16.51) (width 0.38) (layer "B.Cu") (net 2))
 (segment (start 7.112 13.843) (end 7.62 13.335) (width 0.38) (layer "B.Cu") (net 2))
 (segment (start 4.699 26.543) (end 4.699 23.622) (width 0.38) (layer "B.Cu") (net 2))
 (segment (start 3.683004 29.083001) (end 3.683004 28.574998) (width 0.38) (layer "B.Cu") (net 2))
 (segment (start 6.223 9.779) (end 6.223 9.144) (width 0.38) (layer "B.Cu") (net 2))
 (segment (start 14.097 10.16) (end 15.24 10.16) (width 0.38) (layer "B.Cu") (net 2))
 (segment (start 13.208 9.271) (end 14.097 10.16) (width 0.38) (layer "B.Cu") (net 2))
 (segment (start 9.428 33.213) (end 10.133 33.213) (width 0.38) (layer "F.Cu") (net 20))
 (segment (start 10.414 33.494) (end 10.414 35.113) (width 0.38) (layer "F.Cu") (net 20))
 (segment (start 10.414 35.113) (end 11.667999 35.113) (width 0.38) (layer "F.Cu") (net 20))
 (segment (start 10.414 35.113) (end 9.428 35.113) (width 0.38) (layer "F.Cu") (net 20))
 (segment (start 14.686999 38.1) (end 11.683999 35.097) (width 0.38) (layer "F.Cu") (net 20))
 (segment (start 10.133 33.213) (end 10.414 33.494) (width 0.38) (layer "F.Cu") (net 20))
 (segment (start -1.27 38.608) (end -0.381 39.497) (width 0.38) (layer "B.Cu") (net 20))
 (segment (start -0.381 39.497) (end 13.843 39.497) (width 0.38) (layer "B.Cu") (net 20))
 (segment (start -1.27 1.27) (end -1.27 38.608) (width 0.38) (layer "B.Cu") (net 20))
 (segment (start 13.843 39.497) (end 15.24 38.1) (width 0.38) (layer "B.Cu") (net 20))
 (segment (start 0 0) (end -1.27 1.27) (width 0.38) (layer "B.Cu") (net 20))
 (segment (start 8.427 26.461) (end 8.427 25.781) (width 0.38) (layer "F.Cu") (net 1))
 (segment (start 10.558 17.395) (end 10.558 15.847) (width 0.38) (layer "F.Cu") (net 1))
 (segment (start 9.981 12.065) (end 9.991 12.055) (width 0.38) (layer "F.Cu") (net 1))
 (segment (start 6.828 35.113) (end 7.813 35.113) (width 0.38) (layer "F.Cu") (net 1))
 (segment (start 9.477 28.575) (end 9.882 28.17) (width 0.38) (layer "F.Cu") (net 1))
 (segment (start 8.976 12.065) (end 9.981 12.065) (width 0.38) (layer "F.Cu") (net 1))
 (segment (start 8.636 10.414) (end 8.636 9.259) (width 0.38) (layer "F.Cu") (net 1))
 (segment (start 9.882 27.154) (end 9.663 26.935) (width 0.38) (layer "F.Cu") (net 1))
 (segment (start 9.905996 15.748) (end 9.779 15.621004) (width 0.38) (layer "F.Cu") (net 1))
 (segment (start 8.901 26.935) (end 8.427 26.461) (width 0.38) (layer "F.Cu") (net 1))
 (segment (start 8.722 28.575) (end 9.477 28.575) (width 0.38) (layer "F.Cu") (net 1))
 (segment (start 8.760125 8.255) (end 8.760125 9.134875) (width 0.38) (layer "F.Cu") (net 1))
 (segment (start 9.991 12.055) (end 9.991 10.425) (width 0.38) (layer "F.Cu") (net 1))
 (segment (start 6.828 35.113) (end 4.588001 35.113) (width 0.38) (layer "F.Cu") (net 1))
 (segment (start 9.663 26.935) (end 8.901 26.935) (width 0.38) (layer "F.Cu") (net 1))
 (segment (start 9.98 10.414) (end 8.636 10.414) (width 0.38) (layer "F.Cu") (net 1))
 (segment (start 7.813 35.113) (end 7.874 35.052) (width 0.38) (layer "F.Cu") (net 1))
 (segment (start 9.652 25.781) (end 8.427 25.781) (width 0.38) (layer "F.Cu") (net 1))
 (segment (start 9.991 10.425) (end 9.98 10.414) (width 0.38) (layer "F.Cu") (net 1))
 (segment (start 9.882 28.17) (end 9.882 27.154) (width 0.38) (layer "F.Cu") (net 1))
 (segment (start 10.459 15.748) (end 9.905996 15.748) (width 0.38) (layer "F.Cu") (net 1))
 (via (at 9.652 25.781) (size 0.8) (drill 0.4) (layers "F.Cu" "B.Cu") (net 1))
 (via (at 9.779 15.621004) (size 0.8) (drill 0.4) (layers "F.Cu" "B.Cu") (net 1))
 (via (at 7.874 35.052) (size 0.8) (drill 0.4) (layers "F.Cu" "B.Cu") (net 1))
 (via (at 8.760125 8.255) (size 0.8) (drill 0.4) (layers "F.Cu" "B.Cu") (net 1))
 (segment (start 9.779 15.621004) (end 9.779 17.272) (width 0.38) (layer "B.Cu") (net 1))
 (segment (start 9.652 17.399) (end 9.652 25.781) (width 0.38) (layer "B.Cu") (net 1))
 (segment (start 9.779 11.811) (end 8.760125 10.792125) (width 0.38) (layer "B.Cu") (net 1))
 (segment (start 9.779 17.272) (end 9.652 17.399) (width 0.38) (layer "B.Cu") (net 1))
 (segment (start 9.652 33.274) (end 9.652 25.781) (width 0.38) (layer "B.Cu") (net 1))
 (segment (start 9.779 15.621004) (end 9.779 11.811) (width 0.38) (layer "B.Cu") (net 1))
 (segment (start 8.760125 10.792125) (end 8.760125 8.255) (width 0.38) (layer "B.Cu") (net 1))
 (segment (start 7.874 35.052) (end 9.652 33.274) (width 0.38) (layer "B.Cu") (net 1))
 (segment (start 3.455 18.695) (end 4.682 18.695) (width 0.2) (layer "F.Cu") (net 4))
 (segment (start 0 15.24) (end 3.455 18.695) (width 0.2) (layer "F.Cu") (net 4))
 (segment (start 13.335 20.645) (end 10.558 20.645) (width 0.2) (layer "F.Cu") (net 15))
 (segment (start 15.24 20.32) (end 13.66 20.32) (width 0.2) (layer "F.Cu") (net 15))
 (segment (start 13.66 20.32) (end 13.335 20.645) (width 0.2) (layer "F.Cu") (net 15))
 (segment (start 13.97 16.51) (end 15.24 15.24) (width 0.2) (layer "F.Cu") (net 17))
 (segment (start 10.558 19.345) (end 12.532 19.345) (width 0.2) (layer "F.Cu") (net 17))
 (segment (start 12.532 19.345) (end 13.97 17.907) (width 0.2) (layer "F.Cu") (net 17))
 (segment (start 13.97 17.907) (end 13.97 16.51) (width 0.2) (layer "F.Cu") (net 17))
 (segment (start 12.827 16.7135) (end 12.827 10.033) (width 0.2) (layer "F.Cu") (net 19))
 (segment (start 11.4955 18.045) (end 12.827 16.7135) (width 0.2) (layer "F.Cu") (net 19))
 (segment (start 12.827 10.033) (end 15.24 7.62) (width 0.2) (layer "F.Cu") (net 19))
 (segment (start 10.558 18.045) (end 11.4955 18.045) (width 0.2) (layer "F.Cu") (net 19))
 (segment (start 13.675 21.295) (end 10.558 21.295) (width 0.2) (layer "F.Cu") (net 14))
 (segment (start 15.24 22.86) (end 13.675 21.295) (width 0.2) (layer "F.Cu") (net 14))
 (segment (start 4.682 19.345) (end 7.579 19.345) (width 0.2) (layer "F.Cu") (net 5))
 (segment (start 7.579 19.345) (end 7.62 19.304) (width 0.2) (layer "F.Cu") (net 5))
 (segment (start 8.722 29.525) (end 8.722 30.099) (width 0.2) (layer "F.Cu") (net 5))
 (via (at 7.62 19.304) (size 0.8) (drill 0.4) (layers "F.Cu" "B.Cu") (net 5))
 (via (at 8.722 30.099) (size 0.8) (drill 0.4) (layers "F.Cu" "B.Cu") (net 5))
 (segment (start 8.722 25.867) (end 7.62 24.765) (width 0.2) (layer "B.Cu") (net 5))
 (segment (start 8.722 30.099) (end 8.722 25.867) (width 0.2) (layer "B.Cu") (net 5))
 (segment (start 7.62 24.765) (end 7.62 19.304) (width 0.2) (layer "B.Cu") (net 5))
 (segment (start 0 22.86) (end 1.397 22.86) (width 0.2) (layer "F.Cu") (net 8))
 (segment (start 2.962 21.295) (end 4.281 21.295) (width 0.2) (layer "F.Cu") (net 8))
 (segment (start 1.397 22.86) (end 2.962 21.295) (width 0.2) (layer "F.Cu") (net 8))
 (segment (start 8.529 13.462) (end 8.509 13.462) (width 0.2) (layer "F.Cu") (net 3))
 (segment (start 8.976 13.015) (end 8.529 13.462) (width 0.2) (layer "F.Cu") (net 3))
 (segment (start 5.958 18.045) (end 5.969 18.034) (width 0.2) (layer "F.Cu") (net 3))
 (segment (start 4.682 18.045) (end 5.958 18.045) (width 0.2) (layer "F.Cu") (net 3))
 (via (at 8.509 13.462) (size 0.8) (drill 0.4) (layers "F.Cu" "B.Cu") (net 3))
 (via (at 5.969 18.034) (size 0.8) (drill 0.4) (layers "F.Cu" "B.Cu") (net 3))
 (segment (start 8.509 15.494) (end 5.969 18.034) (width 0.2) (layer "B.Cu") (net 3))
 (segment (start 8.509 13.462) (end 8.509 15.494) (width 0.2) (layer "B.Cu") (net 3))
 (segment (start 13.335 17.399) (end 13.335 14.605) (width 0.2) (layer "F.Cu") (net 18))
 (segment (start 10.558 18.695) (end 12.039 18.695) (width 0.2) (layer "F.Cu") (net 18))
 (segment (start 12.039 18.695) (end 13.335 17.399) (width 0.2) (layer "F.Cu") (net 18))
 (segment (start 13.335 14.605) (end 15.24 12.7) (width 0.2) (layer "F.Cu") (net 18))
 (segment (start 12.801 21.945) (end 13.97 23.114) (width 0.2) (layer "F.Cu") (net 13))
 (segment (start 10.558 21.945) (end 12.801 21.945) (width 0.2) (layer "F.Cu") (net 13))
 (segment (start 13.97 24.13) (end 15.24 25.4) (width 0.2) (layer "F.Cu") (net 13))
 (segment (start 13.97 23.114) (end 13.97 24.13) (width 0.2) (layer "F.Cu") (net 13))
 (segment (start 2.413 20.32) (end 2.738 20.645) (width 0.2) (layer "F.Cu") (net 7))
 (segment (start 0 20.32) (end 2.413 20.32) (width 0.2) (layer "F.Cu") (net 7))
 (segment (start 2.738 20.645) (end 4.682 20.645) (width 0.2) (layer "F.Cu") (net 7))
 (segment (start 15.24 30.48) (end 13.208 28.448) (width 0.2) (layer "F.Cu") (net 12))
 (segment (start 12.054 22.595) (end 10.558 22.595) (width 0.2) (layer "F.Cu") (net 12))
 (segment (start 13.208 23.749) (end 12.054 22.595) (width 0.2) (layer "F.Cu") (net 12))
 (segment (start 13.208 28.448) (end 13.208 23.749) (width 0.2) (layer "F.Cu") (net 12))
 (segment (start 10.558 23.245) (end 10.558 23.766) (width 0.2) (layer "F.Cu") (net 11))
 (segment (start 10.558 23.766) (end 10.668 23.876) (width 0.2) (layer "F.Cu") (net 11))
 (via (at 10.668 23.876) (size 0.8) (drill 0.4) (layers "F.Cu" "B.Cu") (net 11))
 (segment (start 7.112 2.54) (end 0 2.54) (width 0.2) (layer "B.Cu") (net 11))
 (segment (start 10.668 6.096) (end 7.112 2.54) (width 0.2) (layer "B.Cu") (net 11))
 (segment (start 10.668 23.876) (end 10.668 6.096) (width 0.2) (layer "B.Cu") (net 11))
 (segment (start 15.24 17.78) (end 13.025 19.995) (width 0.2) (layer "F.Cu") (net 16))
 (segment (start 13.025 19.995) (end 10.558 19.995) (width 0.2) (layer "F.Cu") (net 16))
 (segment (start 0 25.4) (end 3.455 21.945) (width 0.2) (layer "F.Cu") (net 9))
 (segment (start 3.455 21.945) (end 4.281 21.945) (width 0.2) (layer "F.Cu") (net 9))
 (segment (start 3.485 19.995) (end 4.682 19.995) (width 0.2) (layer "F.Cu") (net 6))
 (segment (start 1.27 17.78) (end 3.485 19.995) (width 0.2) (layer "F.Cu") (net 6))
 (segment (start 0 17.78) (end 1.27 17.78) (width 0.2) (layer "F.Cu") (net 6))
 (segment (start 3.621857 22.595) (end 3.175 23.041857) (width 0.2) (layer "F.Cu") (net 10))
 (segment (start 4.281 22.595) (end 3.621857 22.595) (width 0.2) (layer "F.Cu") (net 10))
 (segment (start 3.175 23.041857) (end 3.175 24.257) (width 0.2) (layer "F.Cu") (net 10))
 (via (at 3.175 24.257) (size 0.8) (drill 0.4) (layers "F.Cu" "B.Cu") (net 10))
 (segment (start 0 30.48) (end 3.175 27.305) (width 0.2) (layer "B.Cu") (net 10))
 (segment (start 3.175 27.305) (end 3.175 24.257) (width 0.2) (layer "B.Cu") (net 10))
 (segment (start 8.976 11.115) (end 8.001 11.115) (width 0.2) (layer "F.Cu") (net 21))
 (segment (start 7.055 10.169) (end 5.089 10.169) (width 0.2) (layer "F.Cu") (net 21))
 (segment (start 8.001 11.115) (end 7.055 10.169) (width 0.2) (layer "F.Cu") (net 21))
 (segment (start 5.089 10.169) (end 0 5.08) (width 0.2) (layer "F.Cu") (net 21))
 (segment (start 6.476 13.015) (end 5.549994 13.015) (width 0.2) (layer "F.Cu") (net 22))
 (segment (start 5.549994 13.015) (end 5.460994 12.926) (width 0.2) (layer "F.Cu") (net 22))
 (via (at 5.460994 12.926) (size 0.8) (drill 0.4) (layers "F.Cu" "B.Cu") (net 22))
 (segment (start 5.306 12.926) (end 5.460994 12.926) (width 0.2) (layer "B.Cu") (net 22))
 (segment (start 0 7.62) (end 5.306 12.926) (width 0.2) (layer "B.Cu") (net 22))
 (segment (start 6.476 11.115) (end 1.585 11.115) (width 0.2) (layer "F.Cu") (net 23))
 (segment (start 1.585 11.115) (end 0 12.7) (width 0.2) (layer "F.Cu") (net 23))
 (segment (start 7.065537 27.625) (end 7.065543 27.624994) (width 0.2) (layer "F.Cu") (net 26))
 (segment (start 6.222 27.625) (end 7.065537 27.625) (width 0.2) (layer "F.Cu") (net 26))
 (via (at 7.065543 27.624994) (size 0.8) (drill 0.4) (layers "F.Cu" "B.Cu") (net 26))
 (segment (start 4.191 38.1) (end 7.065543 35.225457) (width 0.2) (layer "B.Cu") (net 26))
 (segment (start 7.065543 35.225457) (end 7.065543 27.624994) (width 0.2) (layer "B.Cu") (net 26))
 (segment (start 0 38.1) (end 4.191 38.1) (width 0.2) (layer "B.Cu") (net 26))
 (segment (start 2.667 30.734) (end 3.876 29.525) (width 0.2) (layer "F.Cu") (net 25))
 (segment (start 2.667 34.036) (end 2.667 30.734) (width 0.2) (layer "F.Cu") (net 25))
 (segment (start 6.222 29.525) (end 3.876 29.525) (width 0.2) (layer "F.Cu") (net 25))
 (segment (start 0 35.56) (end 1.143 35.56) (width 0.2) (layer "F.Cu") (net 25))
 (segment (start 1.143 35.56) (end 2.667 34.036) (width 0.2) (layer "F.Cu") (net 25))
 (segment (start 8.055487 27.625) (end 8.722 27.625) (width 0.2) (layer "F.Cu") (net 24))
 (segment (start 3.81 31.877) (end 5.796048 31.877) (width 0.2) (layer "F.Cu") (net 24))
 (segment (start 5.796048 31.877) (end 7.493 30.180048) (width 0.2) (layer "F.Cu") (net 24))
 (segment (start 7.493 30.180048) (end 7.493 28.187487) (width 0.2) (layer "F.Cu") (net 24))
 (segment (start 7.493 28.187487) (end 8.055487 27.625) (width 0.2) (layer "F.Cu") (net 24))
 (via (at 3.81 31.877) (size 0.8) (drill 0.4) (layers "F.Cu" "B.Cu") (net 24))
 (segment (start 2.159 31.877) (end 1.016 33.02) (width 0.2) (layer "B.Cu") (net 24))
 (segment (start 3.81 31.877) (end 2.159 31.877) (width 0.2) (layer "B.Cu") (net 24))
 (segment (start 1.016 33.02) (end 0 33.02) (width 0.2) (layer "B.Cu") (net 24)))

